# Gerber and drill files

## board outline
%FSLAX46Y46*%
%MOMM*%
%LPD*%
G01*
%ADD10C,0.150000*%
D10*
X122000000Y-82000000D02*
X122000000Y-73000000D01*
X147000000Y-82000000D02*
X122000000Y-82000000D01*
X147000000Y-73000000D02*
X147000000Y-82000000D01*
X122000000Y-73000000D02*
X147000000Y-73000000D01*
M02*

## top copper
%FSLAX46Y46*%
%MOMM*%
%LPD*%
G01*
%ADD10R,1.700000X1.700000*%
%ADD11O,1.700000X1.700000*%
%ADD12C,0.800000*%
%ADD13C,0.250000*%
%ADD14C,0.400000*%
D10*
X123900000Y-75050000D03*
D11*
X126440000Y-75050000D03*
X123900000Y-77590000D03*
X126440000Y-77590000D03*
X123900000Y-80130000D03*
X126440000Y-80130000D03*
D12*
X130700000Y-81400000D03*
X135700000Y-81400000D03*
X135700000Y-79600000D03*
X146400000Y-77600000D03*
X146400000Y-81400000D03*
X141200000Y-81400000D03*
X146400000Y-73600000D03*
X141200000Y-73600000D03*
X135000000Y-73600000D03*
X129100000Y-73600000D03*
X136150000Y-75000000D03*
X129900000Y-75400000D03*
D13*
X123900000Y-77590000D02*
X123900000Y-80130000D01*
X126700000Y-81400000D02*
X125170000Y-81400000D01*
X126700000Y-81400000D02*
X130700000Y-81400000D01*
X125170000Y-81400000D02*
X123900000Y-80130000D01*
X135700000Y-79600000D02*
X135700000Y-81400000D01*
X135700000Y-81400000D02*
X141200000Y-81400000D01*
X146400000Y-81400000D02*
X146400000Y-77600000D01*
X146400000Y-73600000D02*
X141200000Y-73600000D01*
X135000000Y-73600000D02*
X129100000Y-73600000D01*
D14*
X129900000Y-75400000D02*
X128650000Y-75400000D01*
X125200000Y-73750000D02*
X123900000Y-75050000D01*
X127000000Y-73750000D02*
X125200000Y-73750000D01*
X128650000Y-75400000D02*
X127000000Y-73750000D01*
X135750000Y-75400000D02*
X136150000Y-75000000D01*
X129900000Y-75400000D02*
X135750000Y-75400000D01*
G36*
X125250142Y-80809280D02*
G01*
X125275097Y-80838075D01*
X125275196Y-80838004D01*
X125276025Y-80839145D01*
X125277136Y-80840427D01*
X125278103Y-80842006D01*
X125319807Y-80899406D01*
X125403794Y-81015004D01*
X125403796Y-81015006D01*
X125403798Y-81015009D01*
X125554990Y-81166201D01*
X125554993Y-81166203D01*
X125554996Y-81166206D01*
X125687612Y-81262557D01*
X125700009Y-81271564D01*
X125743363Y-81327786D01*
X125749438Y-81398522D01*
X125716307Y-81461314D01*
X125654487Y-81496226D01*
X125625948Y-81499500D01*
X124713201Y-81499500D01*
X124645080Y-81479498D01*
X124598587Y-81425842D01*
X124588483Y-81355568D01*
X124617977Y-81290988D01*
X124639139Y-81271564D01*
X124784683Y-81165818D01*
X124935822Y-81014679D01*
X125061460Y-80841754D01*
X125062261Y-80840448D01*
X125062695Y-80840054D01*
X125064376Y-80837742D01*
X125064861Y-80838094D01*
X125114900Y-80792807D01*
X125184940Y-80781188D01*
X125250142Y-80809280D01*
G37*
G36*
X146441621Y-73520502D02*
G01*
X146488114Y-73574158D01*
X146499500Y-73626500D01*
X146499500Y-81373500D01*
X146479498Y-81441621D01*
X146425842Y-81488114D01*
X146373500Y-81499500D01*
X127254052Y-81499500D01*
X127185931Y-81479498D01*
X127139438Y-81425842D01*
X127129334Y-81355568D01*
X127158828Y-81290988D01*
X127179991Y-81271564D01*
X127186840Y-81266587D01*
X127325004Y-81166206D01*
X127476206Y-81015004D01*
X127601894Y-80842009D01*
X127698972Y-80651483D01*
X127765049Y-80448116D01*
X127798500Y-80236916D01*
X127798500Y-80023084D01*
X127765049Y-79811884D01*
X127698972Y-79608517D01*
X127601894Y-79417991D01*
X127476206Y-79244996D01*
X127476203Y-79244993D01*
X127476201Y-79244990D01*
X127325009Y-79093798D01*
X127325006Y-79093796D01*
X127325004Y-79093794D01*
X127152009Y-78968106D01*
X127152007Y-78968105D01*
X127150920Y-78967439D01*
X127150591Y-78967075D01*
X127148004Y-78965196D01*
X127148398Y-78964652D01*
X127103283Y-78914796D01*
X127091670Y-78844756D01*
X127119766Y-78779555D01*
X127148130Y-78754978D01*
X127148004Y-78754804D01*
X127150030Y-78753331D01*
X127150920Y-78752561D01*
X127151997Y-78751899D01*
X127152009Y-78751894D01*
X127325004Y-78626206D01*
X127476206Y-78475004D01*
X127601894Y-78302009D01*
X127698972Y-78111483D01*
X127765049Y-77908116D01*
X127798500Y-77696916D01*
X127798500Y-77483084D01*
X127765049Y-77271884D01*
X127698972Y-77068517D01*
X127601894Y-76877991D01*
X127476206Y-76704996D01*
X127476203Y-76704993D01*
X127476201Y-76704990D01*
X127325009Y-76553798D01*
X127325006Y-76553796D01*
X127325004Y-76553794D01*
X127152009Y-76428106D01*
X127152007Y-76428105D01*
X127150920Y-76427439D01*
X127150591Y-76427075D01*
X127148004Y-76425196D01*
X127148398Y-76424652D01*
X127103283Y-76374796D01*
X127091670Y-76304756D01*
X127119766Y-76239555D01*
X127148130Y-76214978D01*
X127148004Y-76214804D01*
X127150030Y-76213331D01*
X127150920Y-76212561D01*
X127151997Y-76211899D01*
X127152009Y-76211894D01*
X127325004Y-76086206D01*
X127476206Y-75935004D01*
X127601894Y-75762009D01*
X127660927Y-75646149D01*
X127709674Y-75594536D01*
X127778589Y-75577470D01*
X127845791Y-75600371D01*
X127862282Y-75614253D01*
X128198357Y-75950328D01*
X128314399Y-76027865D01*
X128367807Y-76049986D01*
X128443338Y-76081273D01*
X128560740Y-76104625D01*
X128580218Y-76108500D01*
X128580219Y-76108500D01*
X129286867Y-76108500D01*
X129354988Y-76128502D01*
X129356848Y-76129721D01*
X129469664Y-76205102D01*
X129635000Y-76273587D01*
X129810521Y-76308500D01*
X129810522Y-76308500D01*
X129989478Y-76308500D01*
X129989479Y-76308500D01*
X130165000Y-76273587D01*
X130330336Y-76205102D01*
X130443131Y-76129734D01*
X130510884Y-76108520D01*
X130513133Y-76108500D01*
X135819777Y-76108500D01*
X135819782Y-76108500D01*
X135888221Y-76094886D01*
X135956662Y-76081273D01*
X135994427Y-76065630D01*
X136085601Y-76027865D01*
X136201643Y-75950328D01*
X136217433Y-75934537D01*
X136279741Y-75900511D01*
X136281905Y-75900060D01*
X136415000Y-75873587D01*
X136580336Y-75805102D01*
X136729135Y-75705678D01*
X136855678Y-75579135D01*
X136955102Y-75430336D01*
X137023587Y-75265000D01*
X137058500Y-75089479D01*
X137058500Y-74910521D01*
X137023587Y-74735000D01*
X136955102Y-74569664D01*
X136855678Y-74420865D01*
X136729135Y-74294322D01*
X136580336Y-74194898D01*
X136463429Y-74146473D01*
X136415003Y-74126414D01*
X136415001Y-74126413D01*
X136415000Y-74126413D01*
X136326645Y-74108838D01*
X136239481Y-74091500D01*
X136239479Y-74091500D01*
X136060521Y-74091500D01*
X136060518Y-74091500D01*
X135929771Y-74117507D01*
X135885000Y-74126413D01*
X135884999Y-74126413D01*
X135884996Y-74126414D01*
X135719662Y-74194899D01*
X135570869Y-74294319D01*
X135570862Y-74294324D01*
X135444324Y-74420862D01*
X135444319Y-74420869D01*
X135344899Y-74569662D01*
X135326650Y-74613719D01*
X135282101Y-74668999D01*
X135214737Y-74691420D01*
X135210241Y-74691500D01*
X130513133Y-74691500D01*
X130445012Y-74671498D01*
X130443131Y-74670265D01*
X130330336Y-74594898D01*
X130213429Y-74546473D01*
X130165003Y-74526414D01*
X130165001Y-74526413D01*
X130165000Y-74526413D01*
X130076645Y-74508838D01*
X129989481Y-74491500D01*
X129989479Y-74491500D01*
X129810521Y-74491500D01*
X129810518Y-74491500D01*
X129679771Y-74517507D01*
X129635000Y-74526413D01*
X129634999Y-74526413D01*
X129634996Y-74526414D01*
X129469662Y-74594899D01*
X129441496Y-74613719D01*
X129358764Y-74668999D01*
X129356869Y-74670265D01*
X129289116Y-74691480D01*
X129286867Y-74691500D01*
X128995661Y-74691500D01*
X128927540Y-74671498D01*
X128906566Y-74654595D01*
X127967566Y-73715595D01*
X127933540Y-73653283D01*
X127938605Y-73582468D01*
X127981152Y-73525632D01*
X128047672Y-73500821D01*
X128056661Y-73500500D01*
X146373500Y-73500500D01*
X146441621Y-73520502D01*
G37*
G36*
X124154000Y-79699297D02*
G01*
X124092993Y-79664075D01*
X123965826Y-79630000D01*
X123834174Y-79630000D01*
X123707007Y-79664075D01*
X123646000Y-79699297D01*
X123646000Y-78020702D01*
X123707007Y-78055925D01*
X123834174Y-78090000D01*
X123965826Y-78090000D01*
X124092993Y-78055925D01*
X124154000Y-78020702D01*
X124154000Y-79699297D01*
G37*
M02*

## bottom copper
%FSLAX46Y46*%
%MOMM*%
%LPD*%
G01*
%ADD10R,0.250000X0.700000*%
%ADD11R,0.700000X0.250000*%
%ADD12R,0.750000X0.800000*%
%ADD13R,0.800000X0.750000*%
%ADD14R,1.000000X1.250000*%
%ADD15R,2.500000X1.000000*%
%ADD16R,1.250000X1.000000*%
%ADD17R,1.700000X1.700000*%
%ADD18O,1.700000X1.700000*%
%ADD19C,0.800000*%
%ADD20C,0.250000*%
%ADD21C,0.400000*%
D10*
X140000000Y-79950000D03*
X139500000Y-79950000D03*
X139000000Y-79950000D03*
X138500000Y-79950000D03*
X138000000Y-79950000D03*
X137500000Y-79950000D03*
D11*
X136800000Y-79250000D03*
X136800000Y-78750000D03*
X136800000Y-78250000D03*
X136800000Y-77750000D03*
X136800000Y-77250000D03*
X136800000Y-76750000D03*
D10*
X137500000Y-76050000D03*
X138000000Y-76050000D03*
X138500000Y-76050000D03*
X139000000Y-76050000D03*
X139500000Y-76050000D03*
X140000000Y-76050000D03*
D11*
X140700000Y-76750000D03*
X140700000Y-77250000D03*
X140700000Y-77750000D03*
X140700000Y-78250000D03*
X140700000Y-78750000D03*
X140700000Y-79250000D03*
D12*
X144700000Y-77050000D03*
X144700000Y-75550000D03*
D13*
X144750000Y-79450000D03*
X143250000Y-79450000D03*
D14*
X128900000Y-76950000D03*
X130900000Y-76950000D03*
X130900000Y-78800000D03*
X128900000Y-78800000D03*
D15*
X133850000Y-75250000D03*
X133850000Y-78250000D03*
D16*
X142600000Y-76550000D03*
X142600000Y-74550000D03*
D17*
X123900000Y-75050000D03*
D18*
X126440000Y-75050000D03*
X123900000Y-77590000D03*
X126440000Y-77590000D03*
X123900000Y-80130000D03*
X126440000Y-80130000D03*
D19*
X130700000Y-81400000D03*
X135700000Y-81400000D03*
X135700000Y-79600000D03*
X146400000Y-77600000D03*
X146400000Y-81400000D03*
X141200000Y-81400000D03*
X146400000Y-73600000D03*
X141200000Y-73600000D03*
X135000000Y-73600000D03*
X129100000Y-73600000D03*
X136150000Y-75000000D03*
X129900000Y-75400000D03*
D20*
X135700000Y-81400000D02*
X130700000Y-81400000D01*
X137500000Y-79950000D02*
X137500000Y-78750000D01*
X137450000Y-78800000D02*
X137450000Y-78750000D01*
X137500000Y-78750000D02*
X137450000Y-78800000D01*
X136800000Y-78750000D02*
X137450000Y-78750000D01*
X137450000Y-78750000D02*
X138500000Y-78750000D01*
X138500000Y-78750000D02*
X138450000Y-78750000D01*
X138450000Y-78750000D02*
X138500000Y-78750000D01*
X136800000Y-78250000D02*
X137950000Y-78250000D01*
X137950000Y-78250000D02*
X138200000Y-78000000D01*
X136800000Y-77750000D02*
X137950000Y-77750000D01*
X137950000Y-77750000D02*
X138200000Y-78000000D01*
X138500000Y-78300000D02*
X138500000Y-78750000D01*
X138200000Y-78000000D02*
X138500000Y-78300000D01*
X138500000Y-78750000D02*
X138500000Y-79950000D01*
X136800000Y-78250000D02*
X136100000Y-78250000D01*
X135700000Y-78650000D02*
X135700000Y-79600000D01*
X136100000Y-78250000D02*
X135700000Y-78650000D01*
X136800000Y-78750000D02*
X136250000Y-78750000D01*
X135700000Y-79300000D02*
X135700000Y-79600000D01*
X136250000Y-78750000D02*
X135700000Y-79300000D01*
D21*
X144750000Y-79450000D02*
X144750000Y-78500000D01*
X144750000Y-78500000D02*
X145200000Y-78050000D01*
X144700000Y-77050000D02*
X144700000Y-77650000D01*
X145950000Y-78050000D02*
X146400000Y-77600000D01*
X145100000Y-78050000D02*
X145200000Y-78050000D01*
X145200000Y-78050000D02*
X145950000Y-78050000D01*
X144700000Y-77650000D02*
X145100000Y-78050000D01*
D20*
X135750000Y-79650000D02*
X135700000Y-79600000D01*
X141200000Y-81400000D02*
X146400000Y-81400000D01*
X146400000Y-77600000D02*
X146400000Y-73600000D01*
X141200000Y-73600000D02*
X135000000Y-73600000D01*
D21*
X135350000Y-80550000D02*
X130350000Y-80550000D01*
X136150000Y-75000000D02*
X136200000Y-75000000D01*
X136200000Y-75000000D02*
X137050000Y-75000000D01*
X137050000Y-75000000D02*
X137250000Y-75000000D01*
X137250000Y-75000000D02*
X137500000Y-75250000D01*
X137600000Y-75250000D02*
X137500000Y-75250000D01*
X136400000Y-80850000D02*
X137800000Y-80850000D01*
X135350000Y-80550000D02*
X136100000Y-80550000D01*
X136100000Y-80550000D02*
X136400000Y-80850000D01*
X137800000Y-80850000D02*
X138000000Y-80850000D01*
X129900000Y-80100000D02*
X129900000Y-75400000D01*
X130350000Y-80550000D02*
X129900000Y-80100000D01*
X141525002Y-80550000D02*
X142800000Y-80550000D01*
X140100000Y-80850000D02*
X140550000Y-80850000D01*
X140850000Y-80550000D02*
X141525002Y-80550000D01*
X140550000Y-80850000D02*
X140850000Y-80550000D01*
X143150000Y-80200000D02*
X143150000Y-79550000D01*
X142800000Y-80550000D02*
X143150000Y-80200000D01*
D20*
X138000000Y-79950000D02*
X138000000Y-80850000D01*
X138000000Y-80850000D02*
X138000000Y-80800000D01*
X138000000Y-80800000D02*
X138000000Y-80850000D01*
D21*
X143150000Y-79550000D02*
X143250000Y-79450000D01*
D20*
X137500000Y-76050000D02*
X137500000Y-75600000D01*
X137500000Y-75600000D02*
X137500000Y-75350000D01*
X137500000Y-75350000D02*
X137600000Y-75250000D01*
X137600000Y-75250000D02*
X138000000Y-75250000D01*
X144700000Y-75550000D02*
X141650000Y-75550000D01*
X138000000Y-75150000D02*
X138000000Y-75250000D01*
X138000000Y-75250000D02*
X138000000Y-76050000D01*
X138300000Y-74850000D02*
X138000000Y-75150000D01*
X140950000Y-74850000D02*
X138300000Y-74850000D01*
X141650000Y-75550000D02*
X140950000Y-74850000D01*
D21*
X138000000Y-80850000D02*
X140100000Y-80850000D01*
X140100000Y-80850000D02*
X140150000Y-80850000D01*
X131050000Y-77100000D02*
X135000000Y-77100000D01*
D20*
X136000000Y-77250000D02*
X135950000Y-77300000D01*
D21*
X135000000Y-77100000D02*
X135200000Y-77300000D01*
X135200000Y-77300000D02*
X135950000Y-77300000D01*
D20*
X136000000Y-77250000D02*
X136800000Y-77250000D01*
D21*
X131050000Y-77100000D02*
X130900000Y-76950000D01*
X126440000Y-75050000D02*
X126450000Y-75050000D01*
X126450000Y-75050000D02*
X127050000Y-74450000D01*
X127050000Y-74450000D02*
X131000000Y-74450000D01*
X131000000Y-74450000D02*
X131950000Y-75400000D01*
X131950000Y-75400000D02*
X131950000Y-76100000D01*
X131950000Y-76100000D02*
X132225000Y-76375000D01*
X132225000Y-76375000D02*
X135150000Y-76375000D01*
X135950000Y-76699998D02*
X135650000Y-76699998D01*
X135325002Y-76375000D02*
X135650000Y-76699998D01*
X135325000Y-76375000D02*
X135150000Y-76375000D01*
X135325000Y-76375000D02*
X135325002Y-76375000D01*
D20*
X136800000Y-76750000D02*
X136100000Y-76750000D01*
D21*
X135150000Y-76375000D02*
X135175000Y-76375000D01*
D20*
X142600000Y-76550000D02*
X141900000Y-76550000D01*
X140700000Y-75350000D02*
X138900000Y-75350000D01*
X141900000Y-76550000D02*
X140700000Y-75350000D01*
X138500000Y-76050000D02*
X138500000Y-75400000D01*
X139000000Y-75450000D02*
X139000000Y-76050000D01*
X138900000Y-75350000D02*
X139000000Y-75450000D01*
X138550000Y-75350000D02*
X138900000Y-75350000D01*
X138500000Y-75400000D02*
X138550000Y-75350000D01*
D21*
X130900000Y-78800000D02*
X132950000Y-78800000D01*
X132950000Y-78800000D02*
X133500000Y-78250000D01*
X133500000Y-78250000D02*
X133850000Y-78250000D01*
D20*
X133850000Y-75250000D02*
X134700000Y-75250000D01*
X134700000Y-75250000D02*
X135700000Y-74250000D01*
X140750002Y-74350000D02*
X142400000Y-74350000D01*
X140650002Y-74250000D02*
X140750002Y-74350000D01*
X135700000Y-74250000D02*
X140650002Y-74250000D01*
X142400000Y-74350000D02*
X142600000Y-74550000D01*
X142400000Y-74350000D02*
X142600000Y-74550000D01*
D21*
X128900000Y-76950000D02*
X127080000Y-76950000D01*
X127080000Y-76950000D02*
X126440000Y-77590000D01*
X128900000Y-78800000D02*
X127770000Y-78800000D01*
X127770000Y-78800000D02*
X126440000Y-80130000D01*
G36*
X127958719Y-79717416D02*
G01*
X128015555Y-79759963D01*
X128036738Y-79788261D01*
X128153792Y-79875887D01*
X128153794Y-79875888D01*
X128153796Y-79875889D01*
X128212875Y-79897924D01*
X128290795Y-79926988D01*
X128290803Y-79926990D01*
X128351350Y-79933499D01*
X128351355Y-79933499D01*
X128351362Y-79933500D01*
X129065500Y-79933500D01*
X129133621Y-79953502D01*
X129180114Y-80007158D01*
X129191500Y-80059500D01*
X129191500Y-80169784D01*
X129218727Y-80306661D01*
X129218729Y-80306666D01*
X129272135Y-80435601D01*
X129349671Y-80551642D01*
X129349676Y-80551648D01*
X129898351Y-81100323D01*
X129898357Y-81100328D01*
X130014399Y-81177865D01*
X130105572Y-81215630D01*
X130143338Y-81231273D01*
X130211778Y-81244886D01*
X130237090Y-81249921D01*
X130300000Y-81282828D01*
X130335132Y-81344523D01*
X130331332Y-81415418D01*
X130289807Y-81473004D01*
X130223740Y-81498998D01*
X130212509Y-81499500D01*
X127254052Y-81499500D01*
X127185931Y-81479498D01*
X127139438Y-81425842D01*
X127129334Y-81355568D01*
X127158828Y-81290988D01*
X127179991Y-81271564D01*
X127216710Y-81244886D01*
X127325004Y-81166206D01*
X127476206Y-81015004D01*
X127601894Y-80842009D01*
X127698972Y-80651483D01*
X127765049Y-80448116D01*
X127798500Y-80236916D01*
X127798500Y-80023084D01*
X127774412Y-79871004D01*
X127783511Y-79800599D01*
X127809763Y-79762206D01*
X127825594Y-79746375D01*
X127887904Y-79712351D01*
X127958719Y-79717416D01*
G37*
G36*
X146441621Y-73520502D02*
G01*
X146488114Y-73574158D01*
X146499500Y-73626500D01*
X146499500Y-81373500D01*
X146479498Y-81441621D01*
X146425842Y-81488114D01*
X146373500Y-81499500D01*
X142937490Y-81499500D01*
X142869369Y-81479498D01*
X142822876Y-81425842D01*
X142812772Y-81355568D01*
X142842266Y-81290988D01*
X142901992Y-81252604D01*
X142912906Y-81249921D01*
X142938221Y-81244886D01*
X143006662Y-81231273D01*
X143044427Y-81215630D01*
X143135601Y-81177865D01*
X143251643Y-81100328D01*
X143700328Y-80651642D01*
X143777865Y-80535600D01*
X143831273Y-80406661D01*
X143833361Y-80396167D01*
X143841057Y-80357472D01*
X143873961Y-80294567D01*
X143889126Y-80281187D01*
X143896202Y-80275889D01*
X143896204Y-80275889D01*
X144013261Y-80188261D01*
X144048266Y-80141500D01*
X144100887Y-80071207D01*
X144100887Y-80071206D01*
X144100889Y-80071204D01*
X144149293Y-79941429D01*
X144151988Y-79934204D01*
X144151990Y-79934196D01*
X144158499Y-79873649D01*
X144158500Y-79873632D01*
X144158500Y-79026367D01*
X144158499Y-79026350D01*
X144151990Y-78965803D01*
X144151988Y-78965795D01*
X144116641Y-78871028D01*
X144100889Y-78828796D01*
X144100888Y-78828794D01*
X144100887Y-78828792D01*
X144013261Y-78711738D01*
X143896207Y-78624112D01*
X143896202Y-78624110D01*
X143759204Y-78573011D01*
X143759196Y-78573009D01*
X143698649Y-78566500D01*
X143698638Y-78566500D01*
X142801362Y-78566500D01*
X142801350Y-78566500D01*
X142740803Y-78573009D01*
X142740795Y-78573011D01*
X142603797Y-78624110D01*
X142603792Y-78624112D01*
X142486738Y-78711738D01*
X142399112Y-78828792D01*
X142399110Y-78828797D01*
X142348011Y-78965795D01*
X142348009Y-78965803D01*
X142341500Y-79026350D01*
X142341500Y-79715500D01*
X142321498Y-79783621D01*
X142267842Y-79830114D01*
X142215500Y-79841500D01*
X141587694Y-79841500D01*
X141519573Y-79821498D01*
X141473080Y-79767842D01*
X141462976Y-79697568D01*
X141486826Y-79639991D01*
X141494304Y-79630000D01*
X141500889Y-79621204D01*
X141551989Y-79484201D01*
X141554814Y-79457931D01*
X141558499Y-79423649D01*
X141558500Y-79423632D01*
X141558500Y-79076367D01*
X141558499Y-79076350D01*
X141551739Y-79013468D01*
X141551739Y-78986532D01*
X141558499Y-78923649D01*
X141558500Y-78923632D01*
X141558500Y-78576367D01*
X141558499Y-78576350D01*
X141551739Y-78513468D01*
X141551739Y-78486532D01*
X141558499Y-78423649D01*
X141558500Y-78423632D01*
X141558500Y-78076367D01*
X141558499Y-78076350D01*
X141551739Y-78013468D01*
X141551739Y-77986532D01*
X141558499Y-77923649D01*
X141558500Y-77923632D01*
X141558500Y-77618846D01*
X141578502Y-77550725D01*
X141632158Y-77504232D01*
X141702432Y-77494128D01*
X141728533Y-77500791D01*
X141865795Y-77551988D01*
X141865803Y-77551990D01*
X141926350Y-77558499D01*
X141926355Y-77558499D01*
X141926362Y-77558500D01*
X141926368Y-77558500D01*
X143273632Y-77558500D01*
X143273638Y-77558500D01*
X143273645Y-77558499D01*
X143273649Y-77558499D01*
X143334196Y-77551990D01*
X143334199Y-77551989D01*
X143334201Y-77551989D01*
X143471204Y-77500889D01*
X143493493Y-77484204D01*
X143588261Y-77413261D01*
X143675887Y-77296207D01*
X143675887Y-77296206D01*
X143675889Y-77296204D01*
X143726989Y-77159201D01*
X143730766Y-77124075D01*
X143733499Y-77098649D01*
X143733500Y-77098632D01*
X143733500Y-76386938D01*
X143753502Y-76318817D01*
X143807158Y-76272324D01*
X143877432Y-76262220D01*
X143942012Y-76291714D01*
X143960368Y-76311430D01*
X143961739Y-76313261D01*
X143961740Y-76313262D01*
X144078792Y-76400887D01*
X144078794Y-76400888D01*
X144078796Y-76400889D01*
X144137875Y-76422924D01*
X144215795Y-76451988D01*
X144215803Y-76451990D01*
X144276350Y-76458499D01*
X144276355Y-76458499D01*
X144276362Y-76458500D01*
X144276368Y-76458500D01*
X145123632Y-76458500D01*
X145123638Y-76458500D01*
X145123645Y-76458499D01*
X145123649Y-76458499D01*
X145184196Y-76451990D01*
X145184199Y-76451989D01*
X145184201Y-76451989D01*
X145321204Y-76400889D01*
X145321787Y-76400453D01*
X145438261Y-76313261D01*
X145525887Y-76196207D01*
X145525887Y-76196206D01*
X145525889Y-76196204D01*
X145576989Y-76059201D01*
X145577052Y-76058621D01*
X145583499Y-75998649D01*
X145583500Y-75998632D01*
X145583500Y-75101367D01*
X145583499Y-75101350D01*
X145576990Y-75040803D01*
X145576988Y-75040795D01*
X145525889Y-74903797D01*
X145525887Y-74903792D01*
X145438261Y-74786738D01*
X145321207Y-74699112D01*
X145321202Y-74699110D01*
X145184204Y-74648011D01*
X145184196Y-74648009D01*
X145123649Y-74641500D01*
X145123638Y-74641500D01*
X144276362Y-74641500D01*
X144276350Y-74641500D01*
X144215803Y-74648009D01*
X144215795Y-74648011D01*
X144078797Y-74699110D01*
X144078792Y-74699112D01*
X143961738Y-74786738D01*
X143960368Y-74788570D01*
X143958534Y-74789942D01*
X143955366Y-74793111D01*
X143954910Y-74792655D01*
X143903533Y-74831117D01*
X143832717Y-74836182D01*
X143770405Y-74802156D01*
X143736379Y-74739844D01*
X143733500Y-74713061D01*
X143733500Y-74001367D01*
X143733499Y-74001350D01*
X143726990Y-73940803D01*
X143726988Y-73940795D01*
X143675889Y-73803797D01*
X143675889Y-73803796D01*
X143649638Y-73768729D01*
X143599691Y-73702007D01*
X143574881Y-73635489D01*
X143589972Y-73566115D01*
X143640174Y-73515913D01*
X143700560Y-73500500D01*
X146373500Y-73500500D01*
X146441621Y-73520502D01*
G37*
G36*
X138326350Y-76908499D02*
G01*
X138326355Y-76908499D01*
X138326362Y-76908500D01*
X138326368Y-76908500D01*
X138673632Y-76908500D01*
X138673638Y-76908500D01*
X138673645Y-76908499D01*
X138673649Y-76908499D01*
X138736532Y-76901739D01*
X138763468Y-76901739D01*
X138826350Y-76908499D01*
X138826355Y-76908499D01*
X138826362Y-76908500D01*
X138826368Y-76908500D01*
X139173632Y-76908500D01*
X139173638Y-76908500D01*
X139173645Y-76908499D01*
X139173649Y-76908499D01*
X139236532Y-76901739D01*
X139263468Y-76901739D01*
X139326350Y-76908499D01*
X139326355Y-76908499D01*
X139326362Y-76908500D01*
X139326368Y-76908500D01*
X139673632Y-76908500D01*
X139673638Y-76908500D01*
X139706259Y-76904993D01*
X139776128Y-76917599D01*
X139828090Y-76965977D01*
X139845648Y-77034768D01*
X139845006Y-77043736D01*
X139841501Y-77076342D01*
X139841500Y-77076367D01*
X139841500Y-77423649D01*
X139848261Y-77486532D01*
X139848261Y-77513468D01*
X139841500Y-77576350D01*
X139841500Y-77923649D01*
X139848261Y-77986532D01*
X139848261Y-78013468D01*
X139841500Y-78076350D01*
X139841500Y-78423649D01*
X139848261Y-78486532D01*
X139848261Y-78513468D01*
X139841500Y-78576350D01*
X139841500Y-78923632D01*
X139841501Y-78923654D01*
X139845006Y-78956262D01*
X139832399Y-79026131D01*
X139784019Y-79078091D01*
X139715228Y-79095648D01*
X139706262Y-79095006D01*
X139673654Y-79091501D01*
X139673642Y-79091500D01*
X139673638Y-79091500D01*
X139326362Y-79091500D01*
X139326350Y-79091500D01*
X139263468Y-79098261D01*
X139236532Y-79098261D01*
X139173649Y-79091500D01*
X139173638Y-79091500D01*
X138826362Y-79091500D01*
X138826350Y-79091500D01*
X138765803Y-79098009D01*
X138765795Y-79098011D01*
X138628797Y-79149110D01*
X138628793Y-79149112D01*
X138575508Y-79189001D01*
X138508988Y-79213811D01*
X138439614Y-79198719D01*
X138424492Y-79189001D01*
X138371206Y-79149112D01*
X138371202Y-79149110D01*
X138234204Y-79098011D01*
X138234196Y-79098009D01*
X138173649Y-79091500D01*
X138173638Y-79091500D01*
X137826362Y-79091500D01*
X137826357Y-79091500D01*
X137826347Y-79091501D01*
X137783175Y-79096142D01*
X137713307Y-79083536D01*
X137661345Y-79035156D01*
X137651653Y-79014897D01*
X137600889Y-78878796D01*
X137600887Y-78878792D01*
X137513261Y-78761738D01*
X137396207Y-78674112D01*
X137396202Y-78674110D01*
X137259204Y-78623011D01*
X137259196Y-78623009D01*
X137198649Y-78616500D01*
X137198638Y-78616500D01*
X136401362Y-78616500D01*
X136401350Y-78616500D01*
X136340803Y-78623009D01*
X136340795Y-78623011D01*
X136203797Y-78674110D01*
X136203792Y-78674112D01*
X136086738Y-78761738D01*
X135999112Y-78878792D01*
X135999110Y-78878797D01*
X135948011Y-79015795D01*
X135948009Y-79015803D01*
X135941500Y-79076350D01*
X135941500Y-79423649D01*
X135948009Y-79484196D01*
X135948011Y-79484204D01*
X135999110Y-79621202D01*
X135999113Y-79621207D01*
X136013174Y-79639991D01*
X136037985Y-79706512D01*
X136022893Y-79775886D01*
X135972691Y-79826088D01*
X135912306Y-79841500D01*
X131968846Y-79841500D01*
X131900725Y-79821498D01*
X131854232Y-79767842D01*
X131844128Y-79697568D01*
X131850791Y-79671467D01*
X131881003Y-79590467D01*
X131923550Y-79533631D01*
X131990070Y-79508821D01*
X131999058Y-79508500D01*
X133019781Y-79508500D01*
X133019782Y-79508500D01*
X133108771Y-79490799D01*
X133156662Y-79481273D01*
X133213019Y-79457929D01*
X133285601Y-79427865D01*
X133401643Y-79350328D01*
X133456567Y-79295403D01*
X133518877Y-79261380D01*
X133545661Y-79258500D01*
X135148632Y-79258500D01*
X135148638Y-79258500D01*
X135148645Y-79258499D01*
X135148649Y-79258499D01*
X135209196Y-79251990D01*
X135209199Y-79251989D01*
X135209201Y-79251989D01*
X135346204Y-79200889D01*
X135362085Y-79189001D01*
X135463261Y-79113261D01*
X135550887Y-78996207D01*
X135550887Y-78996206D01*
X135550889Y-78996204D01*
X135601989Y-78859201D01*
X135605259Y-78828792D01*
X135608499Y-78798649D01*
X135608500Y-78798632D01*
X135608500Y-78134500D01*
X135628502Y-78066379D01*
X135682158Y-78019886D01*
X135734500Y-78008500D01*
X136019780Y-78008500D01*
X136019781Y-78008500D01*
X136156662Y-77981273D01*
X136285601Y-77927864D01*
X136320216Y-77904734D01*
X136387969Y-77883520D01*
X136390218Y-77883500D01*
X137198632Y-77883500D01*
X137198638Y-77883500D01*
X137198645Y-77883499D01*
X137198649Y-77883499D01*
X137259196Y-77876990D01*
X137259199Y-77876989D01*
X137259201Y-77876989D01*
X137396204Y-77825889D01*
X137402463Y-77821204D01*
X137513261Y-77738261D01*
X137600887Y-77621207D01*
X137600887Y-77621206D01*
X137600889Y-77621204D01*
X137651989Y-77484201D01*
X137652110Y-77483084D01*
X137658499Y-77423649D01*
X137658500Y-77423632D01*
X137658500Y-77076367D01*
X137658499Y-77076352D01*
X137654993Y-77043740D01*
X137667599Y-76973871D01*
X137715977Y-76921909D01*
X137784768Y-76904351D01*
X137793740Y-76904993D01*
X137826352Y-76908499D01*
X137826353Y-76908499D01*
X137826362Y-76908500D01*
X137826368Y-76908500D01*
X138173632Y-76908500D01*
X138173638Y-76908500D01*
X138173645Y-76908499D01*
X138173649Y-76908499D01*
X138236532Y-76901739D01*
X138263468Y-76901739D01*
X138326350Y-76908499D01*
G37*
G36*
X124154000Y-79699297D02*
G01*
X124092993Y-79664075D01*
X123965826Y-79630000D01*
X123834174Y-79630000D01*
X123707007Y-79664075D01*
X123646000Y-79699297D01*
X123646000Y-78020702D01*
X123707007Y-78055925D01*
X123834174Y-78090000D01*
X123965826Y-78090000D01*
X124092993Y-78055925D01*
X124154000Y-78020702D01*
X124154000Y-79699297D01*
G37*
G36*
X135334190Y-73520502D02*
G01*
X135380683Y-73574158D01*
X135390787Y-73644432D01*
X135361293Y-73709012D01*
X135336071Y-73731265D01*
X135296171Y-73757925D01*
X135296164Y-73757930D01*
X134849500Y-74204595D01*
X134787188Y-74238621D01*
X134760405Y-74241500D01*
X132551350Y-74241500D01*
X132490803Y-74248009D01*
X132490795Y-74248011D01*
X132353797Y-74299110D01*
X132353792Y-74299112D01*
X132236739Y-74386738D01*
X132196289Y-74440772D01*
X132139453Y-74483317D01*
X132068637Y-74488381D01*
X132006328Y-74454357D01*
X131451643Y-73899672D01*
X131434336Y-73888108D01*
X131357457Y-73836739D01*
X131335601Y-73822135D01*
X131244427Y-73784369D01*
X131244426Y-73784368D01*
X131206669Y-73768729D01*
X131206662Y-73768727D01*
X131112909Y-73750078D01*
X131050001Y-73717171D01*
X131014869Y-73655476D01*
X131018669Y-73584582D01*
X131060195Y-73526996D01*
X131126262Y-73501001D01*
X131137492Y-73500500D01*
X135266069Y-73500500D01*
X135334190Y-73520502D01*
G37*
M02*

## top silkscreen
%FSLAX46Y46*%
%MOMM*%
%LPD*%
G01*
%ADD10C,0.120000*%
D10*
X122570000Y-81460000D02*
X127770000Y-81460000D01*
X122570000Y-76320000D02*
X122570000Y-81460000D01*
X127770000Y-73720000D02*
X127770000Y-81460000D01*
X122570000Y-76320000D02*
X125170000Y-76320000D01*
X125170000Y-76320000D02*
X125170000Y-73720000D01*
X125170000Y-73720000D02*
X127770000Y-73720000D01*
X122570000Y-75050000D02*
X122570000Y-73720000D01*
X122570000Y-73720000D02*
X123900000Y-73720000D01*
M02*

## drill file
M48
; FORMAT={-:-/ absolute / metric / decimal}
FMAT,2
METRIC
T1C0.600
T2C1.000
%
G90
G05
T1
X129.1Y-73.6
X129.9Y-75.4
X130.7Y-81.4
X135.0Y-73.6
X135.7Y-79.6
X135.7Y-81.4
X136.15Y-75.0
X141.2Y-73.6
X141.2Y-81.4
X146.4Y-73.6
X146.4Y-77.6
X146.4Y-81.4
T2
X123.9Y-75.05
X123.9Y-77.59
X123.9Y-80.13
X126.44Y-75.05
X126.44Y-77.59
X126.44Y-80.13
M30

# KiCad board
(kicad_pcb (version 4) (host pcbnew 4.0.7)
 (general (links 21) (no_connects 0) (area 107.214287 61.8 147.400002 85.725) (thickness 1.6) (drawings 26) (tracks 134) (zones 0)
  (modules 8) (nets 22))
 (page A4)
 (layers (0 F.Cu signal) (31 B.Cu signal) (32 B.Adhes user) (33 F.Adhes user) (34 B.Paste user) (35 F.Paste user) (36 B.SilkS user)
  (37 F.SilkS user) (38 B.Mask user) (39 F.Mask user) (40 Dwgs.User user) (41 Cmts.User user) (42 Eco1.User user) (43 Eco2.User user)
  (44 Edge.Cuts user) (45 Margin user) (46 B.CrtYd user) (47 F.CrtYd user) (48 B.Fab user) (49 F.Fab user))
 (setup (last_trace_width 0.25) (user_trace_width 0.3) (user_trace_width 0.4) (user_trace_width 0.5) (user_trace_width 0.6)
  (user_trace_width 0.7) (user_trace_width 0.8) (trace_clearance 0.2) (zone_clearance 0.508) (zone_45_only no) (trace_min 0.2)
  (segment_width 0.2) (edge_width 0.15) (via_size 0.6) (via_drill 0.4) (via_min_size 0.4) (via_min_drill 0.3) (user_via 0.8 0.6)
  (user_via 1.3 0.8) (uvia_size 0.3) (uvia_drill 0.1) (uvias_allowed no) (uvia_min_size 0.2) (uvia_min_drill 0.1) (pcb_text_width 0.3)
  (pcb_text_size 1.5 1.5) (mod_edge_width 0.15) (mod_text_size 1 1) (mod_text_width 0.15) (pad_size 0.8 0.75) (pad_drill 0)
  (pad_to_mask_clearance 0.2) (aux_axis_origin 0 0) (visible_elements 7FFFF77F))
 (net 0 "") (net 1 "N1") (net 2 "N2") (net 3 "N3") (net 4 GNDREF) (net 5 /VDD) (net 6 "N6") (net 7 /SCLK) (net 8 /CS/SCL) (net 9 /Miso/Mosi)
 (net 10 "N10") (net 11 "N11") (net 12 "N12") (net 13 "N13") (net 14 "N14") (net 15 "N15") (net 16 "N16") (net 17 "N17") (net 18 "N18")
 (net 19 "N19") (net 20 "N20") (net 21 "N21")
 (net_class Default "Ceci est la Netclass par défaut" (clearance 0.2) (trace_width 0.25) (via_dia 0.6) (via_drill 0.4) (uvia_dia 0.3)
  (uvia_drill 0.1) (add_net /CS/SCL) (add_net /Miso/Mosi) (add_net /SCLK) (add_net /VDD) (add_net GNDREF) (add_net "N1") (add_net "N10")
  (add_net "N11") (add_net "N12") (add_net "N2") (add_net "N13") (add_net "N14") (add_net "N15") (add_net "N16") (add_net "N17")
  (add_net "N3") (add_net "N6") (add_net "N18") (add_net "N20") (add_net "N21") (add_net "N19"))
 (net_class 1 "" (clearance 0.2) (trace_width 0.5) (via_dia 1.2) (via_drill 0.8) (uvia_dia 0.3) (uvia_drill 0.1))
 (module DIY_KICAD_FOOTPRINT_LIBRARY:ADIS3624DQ (layer B.Cu) (at 138.75 78 90)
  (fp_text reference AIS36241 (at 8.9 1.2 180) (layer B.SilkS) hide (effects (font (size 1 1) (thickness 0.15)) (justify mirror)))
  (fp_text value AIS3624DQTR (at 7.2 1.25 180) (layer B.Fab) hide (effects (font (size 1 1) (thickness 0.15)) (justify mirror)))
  (pad 1 smd rect (at -1.95 1.25 90) (size 0.7 0.25) (layers B.Cu B.Paste B.Mask) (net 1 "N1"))
  (pad 2 smd rect (at -1.95 0.75 90) (size 0.7 0.25) (layers B.Cu B.Paste B.Mask) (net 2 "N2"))
  (pad 3 smd rect (at -1.95 0.25 90) (size 0.7 0.25) (layers B.Cu B.Paste B.Mask) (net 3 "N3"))
  (pad 4 smd rect (at -1.95 -0.25 90) (size 0.7 0.25) (layers B.Cu B.Paste B.Mask) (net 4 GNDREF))
  (pad 5 smd rect (at -1.95 -0.75 90) (size 0.7 0.25) (layers B.Cu B.Paste B.Mask) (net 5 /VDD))
  (pad 6 smd rect (at -1.95 -1.25 90) (size 0.7 0.25) (layers B.Cu B.Paste B.Mask) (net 4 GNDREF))
  (pad 7 smd rect (at -1.25 -1.95 180) (size 0.7 0.25) (layers B.Cu B.Paste B.Mask) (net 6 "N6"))
  (pad 8 smd rect (at -0.75 -1.95 180) (size 0.7 0.25) (layers B.Cu B.Paste B.Mask) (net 4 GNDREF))
  (pad 9 smd rect (at -0.25 -1.95 180) (size 0.7 0.25) (layers B.Cu B.Paste B.Mask) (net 4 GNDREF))
  (pad 10 smd rect (at 0.25 -1.95 180) (size 0.7 0.25) (layers B.Cu B.Paste B.Mask) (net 4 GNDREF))
  (pad 11 smd rect (at 0.75 -1.95 180) (size 0.7 0.25) (layers B.Cu B.Paste B.Mask) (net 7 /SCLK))
  (pad 12 smd rect (at 1.25 -1.95 180) (size 0.7 0.25) (layers B.Cu B.Paste B.Mask) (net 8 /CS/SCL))
  (pad 13 smd rect (at 1.95 -1.25 90) (size 0.7 0.25) (layers B.Cu B.Paste B.Mask) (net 5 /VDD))
  (pad 14 smd rect (at 1.95 -0.75 90) (size 0.7 0.25) (layers B.Cu B.Paste B.Mask) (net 5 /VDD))
  (pad 15 smd rect (at 1.95 -0.25 90) (size 0.7 0.25) (layers B.Cu B.Paste B.Mask) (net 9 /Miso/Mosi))
  (pad 16 smd rect (at 1.95 0.25 90) (size 0.7 0.25) (layers B.Cu B.Paste B.Mask) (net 9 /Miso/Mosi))
  (pad 17 smd rect (at 1.95 0.75 90) (size 0.7 0.25) (layers B.Cu B.Paste B.Mask) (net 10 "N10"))
  (pad 18 smd rect (at 1.95 1.25 90) (size 0.7 0.25) (layers B.Cu B.Paste B.Mask) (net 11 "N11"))
  (pad 19 smd rect (at 1.25 1.95) (size 0.7 0.25) (layers B.Cu B.Paste B.Mask) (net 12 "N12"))
  (pad 20 smd rect (at 0.75 1.95) (size 0.7 0.25) (layers B.Cu B.Paste B.Mask) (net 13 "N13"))
  (pad 21 smd rect (at 0.25 1.95) (size 0.7 0.25) (layers B.Cu B.Paste B.Mask) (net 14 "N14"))
  (pad 22 smd rect (at -0.25 1.95) (size 0.7 0.25) (layers B.Cu B.Paste B.Mask) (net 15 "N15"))
  (pad 23 smd rect (at -0.75 1.95) (size 0.7 0.25) (layers B.Cu B.Paste B.Mask) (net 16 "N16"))
  (pad 24 smd rect (at -1.25 1.95) (size 0.7 0.25) (layers B.Cu B.Paste B.Mask) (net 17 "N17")))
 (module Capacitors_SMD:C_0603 (layer B.Cu) (at 144.7 76.3 270)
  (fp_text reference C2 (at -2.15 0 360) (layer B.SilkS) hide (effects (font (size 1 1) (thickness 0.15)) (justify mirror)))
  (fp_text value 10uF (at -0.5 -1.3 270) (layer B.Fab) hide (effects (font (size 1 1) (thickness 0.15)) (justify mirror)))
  (pad 2 smd rect (at 0.75 0 270) (size 0.8 0.75) (layers B.Cu B.Paste B.Mask) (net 4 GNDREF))
  (pad 1 smd rect (at -0.75 0 270) (size 0.8 0.75) (layers B.Cu B.Paste B.Mask) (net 5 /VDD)))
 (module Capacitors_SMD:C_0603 (layer B.Cu) (at 144 79.45)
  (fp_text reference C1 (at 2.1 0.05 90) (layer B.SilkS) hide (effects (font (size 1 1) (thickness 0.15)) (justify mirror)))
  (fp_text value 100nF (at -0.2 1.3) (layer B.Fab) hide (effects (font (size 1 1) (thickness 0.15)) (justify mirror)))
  (pad 2 smd rect (at 0.75 0) (size 0.8 0.75) (layers B.Cu B.Paste B.Mask) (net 4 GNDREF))
  (pad 1 smd rect (at -0.75 0) (size 0.8 0.75) (layers B.Cu B.Paste B.Mask) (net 5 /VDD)))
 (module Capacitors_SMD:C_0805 (layer B.Cu) (at 129.9 76.95)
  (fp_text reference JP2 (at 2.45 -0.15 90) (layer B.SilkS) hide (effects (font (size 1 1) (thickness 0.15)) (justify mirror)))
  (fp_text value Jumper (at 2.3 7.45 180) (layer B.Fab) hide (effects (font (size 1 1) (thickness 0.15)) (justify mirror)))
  (pad 1 smd rect (at -1 0) (size 1 1.25) (layers B.Cu B.Paste B.Mask) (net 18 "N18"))
  (pad 2 smd rect (at 1 0) (size 1 1.25) (layers B.Cu B.Paste B.Mask) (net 7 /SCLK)))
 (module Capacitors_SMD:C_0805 (layer B.Cu) (at 129.9 78.8 180)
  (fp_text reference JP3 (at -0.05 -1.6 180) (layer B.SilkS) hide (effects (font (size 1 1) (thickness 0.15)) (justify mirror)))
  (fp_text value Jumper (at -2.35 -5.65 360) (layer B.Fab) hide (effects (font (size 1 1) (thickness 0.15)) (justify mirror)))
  (pad 1 smd rect (at -1 0 180) (size 1 1.25) (layers B.Cu B.Paste B.Mask) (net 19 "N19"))
  (pad 2 smd rect (at 1 0 180) (size 1 1.25) (layers B.Cu B.Paste B.Mask) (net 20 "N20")))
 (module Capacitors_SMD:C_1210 (layer B.Cu) (at 133.85 76.75 270)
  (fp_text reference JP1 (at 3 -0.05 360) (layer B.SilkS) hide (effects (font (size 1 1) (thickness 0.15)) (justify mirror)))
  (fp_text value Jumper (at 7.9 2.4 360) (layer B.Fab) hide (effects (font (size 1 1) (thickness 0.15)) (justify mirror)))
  (pad 1 smd rect (at -1.5 0 270) (size 1 2.5) (layers B.Cu B.Paste B.Mask) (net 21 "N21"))
  (pad 2 smd rect (at 1.5 0 270) (size 1 2.5) (layers B.Cu B.Paste B.Mask) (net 19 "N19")))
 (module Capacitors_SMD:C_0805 (layer B.Cu) (at 142.6 75.55 90)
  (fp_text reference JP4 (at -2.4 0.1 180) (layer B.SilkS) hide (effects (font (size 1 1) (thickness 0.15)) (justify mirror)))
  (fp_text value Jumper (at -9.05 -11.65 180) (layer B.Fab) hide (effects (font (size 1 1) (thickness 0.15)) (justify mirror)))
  (pad 1 smd rect (at -1 0 90) (size 1 1.25) (layers B.Cu B.Paste B.Mask) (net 9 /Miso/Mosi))
  (pad 2 smd rect (at 1 0 90) (size 1 1.25) (layers B.Cu B.Paste B.Mask) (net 21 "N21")))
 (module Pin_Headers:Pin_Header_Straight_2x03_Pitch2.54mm (layer F.Cu) (at 123.9 75.05)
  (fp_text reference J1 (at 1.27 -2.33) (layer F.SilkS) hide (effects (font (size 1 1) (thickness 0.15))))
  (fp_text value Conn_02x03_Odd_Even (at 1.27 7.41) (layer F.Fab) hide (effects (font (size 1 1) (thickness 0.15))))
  (fp_line (start -1.33 6.41) (end 3.87 6.41) (layer F.SilkS) (width 0.12))
  (fp_line (start -1.33 1.27) (end -1.33 6.41) (layer F.SilkS) (width 0.12))
  (fp_line (start 3.87 -1.33) (end 3.87 6.41) (layer F.SilkS) (width 0.12))
  (fp_line (start -1.33 1.27) (end 1.27 1.27) (layer F.SilkS) (width 0.12))
  (fp_line (start 1.27 1.27) (end 1.27 -1.33) (layer F.SilkS) (width 0.12))
  (fp_line (start 1.27 -1.33) (end 3.87 -1.33) (layer F.SilkS) (width 0.12))
  (fp_line (start -1.33 0) (end -1.33 -1.33) (layer F.SilkS) (width 0.12))
  (fp_line (start -1.33 -1.33) (end 0 -1.33) (layer F.SilkS) (width 0.12))
  (pad 1 thru_hole rect (at 0 0) (size 1.7 1.7) (drill 1) (layers *.Cu *.Mask) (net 5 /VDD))
  (pad 2 thru_hole oval (at 2.54 0) (size 1.7 1.7) (drill 1) (layers *.Cu *.Mask) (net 8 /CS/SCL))
  (pad 3 thru_hole oval (at 0 2.54) (size 1.7 1.7) (drill 1) (layers *.Cu *.Mask) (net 4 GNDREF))
  (pad 4 thru_hole oval (at 2.54 2.54) (size 1.7 1.7) (drill 1) (layers *.Cu *.Mask) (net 18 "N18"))
  (pad 5 thru_hole oval (at 0 5.08) (size 1.7 1.7) (drill 1) (layers *.Cu *.Mask) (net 4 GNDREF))
  (pad 6 thru_hole oval (at 2.54 5.08) (size 1.7 1.7) (drill 1) (layers *.Cu *.Mask) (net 20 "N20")))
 (gr_line (start 122 82) (end 122 73) (angle 90) (layer Edge.Cuts) (width 0.15))
 (gr_line (start 147 82) (end 122 82) (angle 90) (layer Edge.Cuts) (width 0.15))
 (gr_line (start 147 73) (end 147 82) (angle 90) (layer Edge.Cuts) (width 0.15))
 (gr_line (start 122 73) (end 147 73) (angle 90) (layer Edge.Cuts) (width 0.15))
 (segment (start 123.9 77.59) (end 123.9 80.13) (width 0.25) (layer F.Cu) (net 4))
 (segment (start 126.7 81.4) (end 125.17 81.4) (width 0.25) (layer F.Cu) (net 4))
 (segment (start 126.7 81.4) (end 130.7 81.4) (width 0.25) (layer F.Cu) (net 4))
 (via (at 130.7 81.4) (size 0.8) (drill 0.6) (layers F.Cu B.Cu) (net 4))
 (segment (start 135.7 81.4) (end 130.7 81.4) (width 0.25) (layer B.Cu) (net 4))
 (via (at 135.7 81.4) (size 0.8) (drill 0.6) (layers F.Cu B.Cu) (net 4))
 (segment (start 125.17 81.4) (end 123.9 80.13) (width 0.25) (layer F.Cu) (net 4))
 (segment (start 137.5 79.95) (end 137.5 78.75) (width 0.25) (layer B.Cu) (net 4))
 (segment (start 137.45 78.8) (end 137.45 78.75) (width 0.25) (layer B.Cu) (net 4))
 (segment (start 137.5 78.75) (end 137.45 78.8) (width 0.25) (layer B.Cu) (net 4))
 (segment (start 136.8 78.75) (end 137.45 78.75) (width 0.25) (layer B.Cu) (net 4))
 (segment (start 137.45 78.75) (end 138.5 78.75) (width 0.25) (layer B.Cu) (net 4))
 (segment (start 138.5 78.75) (end 138.45 78.75) (width 0.25) (layer B.Cu) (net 4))
 (segment (start 138.45 78.75) (end 138.5 78.75) (width 0.25) (layer B.Cu) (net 4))
 (segment (start 136.8 78.25) (end 137.95 78.25) (width 0.25) (layer B.Cu) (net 4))
 (segment (start 137.95 78.25) (end 138.2 78) (width 0.25) (layer B.Cu) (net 4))
 (segment (start 136.8 77.75) (end 137.95 77.75) (width 0.25) (layer B.Cu) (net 4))
 (segment (start 137.95 77.75) (end 138.2 78) (width 0.25) (layer B.Cu) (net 4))
 (segment (start 138.5 78.3) (end 138.5 78.75) (width 0.25) (layer B.Cu) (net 4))
 (segment (start 138.2 78) (end 138.5 78.3) (width 0.25) (layer B.Cu) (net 4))
 (segment (start 138.5 78.75) (end 138.5 79.95) (width 0.25) (layer B.Cu) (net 4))
 (segment (start 136.8 78.25) (end 136.1 78.25) (width 0.25) (layer B.Cu) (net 4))
 (segment (start 135.7 78.65) (end 135.7 79.6) (width 0.25) (layer B.Cu) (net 4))
 (segment (start 136.1 78.25) (end 135.7 78.65) (width 0.25) (layer B.Cu) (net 4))
 (segment (start 136.8 78.75) (end 136.25 78.75) (width 0.25) (layer B.Cu) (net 4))
 (segment (start 135.7 79.3) (end 135.7 79.6) (width 0.25) (layer B.Cu) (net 4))
 (segment (start 136.25 78.75) (end 135.7 79.3) (width 0.25) (layer B.Cu) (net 4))
 (segment (start 144.75 79.45) (end 144.75 78.5) (width 0.4) (layer B.Cu) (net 4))
 (segment (start 144.75 78.5) (end 145.2 78.05) (width 0.4) (layer B.Cu) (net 4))
 (segment (start 144.7 77.05) (end 144.7 77.65) (width 0.4) (layer B.Cu) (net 4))
 (segment (start 145.95 78.05) (end 146.4 77.6) (width 0.4) (layer B.Cu) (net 4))
 (segment (start 145.1 78.05) (end 145.2 78.05) (width 0.4) (layer B.Cu) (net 4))
 (segment (start 145.2 78.05) (end 145.95 78.05) (width 0.4) (layer B.Cu) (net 4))
 (segment (start 144.7 77.65) (end 145.1 78.05) (width 0.4) (layer B.Cu) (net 4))
 (segment (start 135.75 79.65) (end 135.7 79.6) (width 0.25) (layer B.Cu) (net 4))
 (via (at 135.7 79.6) (size 0.8) (drill 0.6) (layers F.Cu B.Cu) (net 4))
 (segment (start 135.7 79.6) (end 135.7 81.4) (width 0.25) (layer F.Cu) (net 4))
 (segment (start 135.7 81.4) (end 141.2 81.4) (width 0.25) (layer F.Cu) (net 4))
 (via (at 146.4 77.6) (size 0.8) (drill 0.6) (layers F.Cu B.Cu) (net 4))
 (segment (start 146.4 81.4) (end 146.4 77.6) (width 0.25) (layer F.Cu) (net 4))
 (via (at 146.4 81.4) (size 0.8) (drill 0.6) (layers F.Cu B.Cu) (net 4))
 (segment (start 141.2 81.4) (end 146.4 81.4) (width 0.25) (layer B.Cu) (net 4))
 (via (at 141.2 81.4) (size 0.8) (drill 0.6) (layers F.Cu B.Cu) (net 4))
 (segment (start 146.4 77.6) (end 146.4 73.6) (width 0.25) (layer B.Cu) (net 4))
 (via (at 146.4 73.6) (size 0.8) (drill 0.6) (layers F.Cu B.Cu) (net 4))
 (segment (start 146.4 73.6) (end 141.2 73.6) (width 0.25) (layer F.Cu) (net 4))
 (via (at 141.2 73.6) (size 0.8) (drill 0.6) (layers F.Cu B.Cu) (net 4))
 (segment (start 141.2 73.6) (end 135 73.6) (width 0.25) (layer B.Cu) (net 4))
 (via (at 135 73.6) (size 0.8) (drill 0.6) (layers F.Cu B.Cu) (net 4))
 (segment (start 135 73.6) (end 129.1 73.6) (width 0.25) (layer F.Cu) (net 4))
 (via (at 129.1 73.6) (size 0.8) (drill 0.6) (layers F.Cu B.Cu) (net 4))
 (segment (start 129.9 75.4) (end 128.65 75.4) (width 0.4) (layer F.Cu) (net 5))
 (segment (start 125.2 73.75) (end 123.9 75.05) (width 0.4) (layer F.Cu) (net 5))
 (segment (start 127 73.75) (end 125.2 73.75) (width 0.4) (layer F.Cu) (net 5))
 (segment (start 128.65 75.4) (end 127 73.75) (width 0.4) (layer F.Cu) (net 5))
 (segment (start 135.35 80.55) (end 130.35 80.55) (width 0.4) (layer B.Cu) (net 5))
 (segment (start 135.75 75.4) (end 136.15 75) (width 0.4) (layer F.Cu) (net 5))
 (via (at 136.15 75) (size 0.8) (drill 0.6) (layers F.Cu B.Cu) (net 5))
 (segment (start 136.15 75) (end 136.2 75) (width 0.4) (layer B.Cu) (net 5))
 (segment (start 136.2 75) (end 137.05 75) (width 0.4) (layer B.Cu) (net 5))
 (segment (start 137.05 75) (end 137.25 75) (width 0.4) (layer B.Cu) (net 5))
 (segment (start 137.25 75) (end 137.5 75.25) (width 0.4) (layer B.Cu) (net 5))
 (segment (start 137.6 75.25) (end 137.5 75.25) (width 0.4) (layer B.Cu) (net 5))
 (segment (start 136.4 80.85) (end 137.8 80.85) (width 0.4) (layer B.Cu) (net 5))
 (segment (start 135.35 80.55) (end 136.1 80.55) (width 0.4) (layer B.Cu) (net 5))
 (segment (start 136.1 80.55) (end 136.4 80.85) (width 0.4) (layer B.Cu) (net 5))
 (segment (start 137.8 80.85) (end 138 80.85) (width 0.4) (layer B.Cu) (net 5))
 (segment (start 129.9 75.4) (end 135.75 75.4) (width 0.4) (layer F.Cu) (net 5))
 (via (at 129.9 75.4) (size 0.8) (drill 0.6) (layers F.Cu B.Cu) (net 5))
 (segment (start 129.9 80.1) (end 129.9 75.4) (width 0.4) (layer B.Cu) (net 5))
 (segment (start 130.35 80.55) (end 129.9 80.1) (width 0.4) (layer B.Cu) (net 5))
 (segment (start 141.525002 80.55) (end 142.8 80.55) (width 0.4) (layer B.Cu) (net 5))
 (segment (start 140.1 80.85) (end 140.55 80.85) (width 0.4) (layer B.Cu) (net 5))
 (segment (start 140.85 80.55) (end 141.525002 80.55) (width 0.4) (layer B.Cu) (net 5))
 (segment (start 140.55 80.85) (end 140.85 80.55) (width 0.4) (layer B.Cu) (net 5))
 (segment (start 143.15 80.2) (end 143.15 79.55) (width 0.4) (layer B.Cu) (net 5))
 (segment (start 142.8 80.55) (end 143.15 80.2) (width 0.4) (layer B.Cu) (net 5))
 (segment (start 138 79.95) (end 138 80.85) (width 0.25) (layer B.Cu) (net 5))
 (segment (start 138 80.85) (end 138 80.8) (width 0.25) (layer B.Cu) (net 5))
 (segment (start 138 80.8) (end 138 80.85) (width 0.25) (layer B.Cu) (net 5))
 (segment (start 143.15 79.55) (end 143.25 79.45) (width 0.4) (layer B.Cu) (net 5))
 (segment (start 137.5 76.05) (end 137.5 75.6) (width 0.25) (layer B.Cu) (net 5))
 (segment (start 137.5 75.6) (end 137.5 75.35) (width 0.25) (layer B.Cu) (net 5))
 (segment (start 137.5 75.35) (end 137.6 75.25) (width 0.25) (layer B.Cu) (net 5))
 (segment (start 137.6 75.25) (end 138 75.25) (width 0.25) (layer B.Cu) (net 5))
 (segment (start 144.7 75.55) (end 141.65 75.55) (width 0.25) (layer B.Cu) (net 5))
 (segment (start 138 75.15) (end 138 75.25) (width 0.25) (layer B.Cu) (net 5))
 (segment (start 138 75.25) (end 138 76.05) (width 0.25) (layer B.Cu) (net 5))
 (segment (start 138.3 74.85) (end 138 75.15) (width 0.25) (layer B.Cu) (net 5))
 (segment (start 140.95 74.85) (end 138.3 74.85) (width 0.25) (layer B.Cu) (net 5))
 (segment (start 141.65 75.55) (end 140.95 74.85) (width 0.25) (layer B.Cu) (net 5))
 (segment (start 138 80.85) (end 140.1 80.85) (width 0.4) (layer B.Cu) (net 5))
 (segment (start 140.1 80.85) (end 140.15 80.85) (width 0.4) (layer B.Cu) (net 5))
 (segment (start 131.05 77.1) (end 135 77.1) (width 0.4) (layer B.Cu) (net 7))
 (segment (start 136 77.25) (end 135.95 77.3) (width 0.25) (layer B.Cu) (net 7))
 (segment (start 135 77.1) (end 135.2 77.3) (width 0.4) (layer B.Cu) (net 7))
 (segment (start 135.2 77.3) (end 135.95 77.3) (width 0.4) (layer B.Cu) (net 7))
 (segment (start 136 77.25) (end 136.8 77.25) (width 0.25) (layer B.Cu) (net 7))
 (segment (start 131.05 77.1) (end 130.9 76.95) (width 0.4) (layer B.Cu) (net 7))
 (segment (start 126.44 75.05) (end 126.45 75.05) (width 0.4) (layer B.Cu) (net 8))
 (segment (start 126.45 75.05) (end 127.05 74.45) (width 0.4) (layer B.Cu) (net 8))
 (segment (start 127.05 74.45) (end 131 74.45) (width 0.4) (layer B.Cu) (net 8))
 (segment (start 131 74.45) (end 131.95 75.4) (width 0.4) (layer B.Cu) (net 8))
 (segment (start 131.95 75.4) (end 131.95 76.1) (width 0.4) (layer B.Cu) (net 8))
 (segment (start 131.95 76.1) (end 132.225 76.375) (width 0.4) (layer B.Cu) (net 8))
 (segment (start 132.225 76.375) (end 135.15 76.375) (width 0.4) (layer B.Cu) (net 8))
 (segment (start 135.95 76.699998) (end 135.65 76.699998) (width 0.4) (layer B.Cu) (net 8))
 (segment (start 135.325002 76.375) (end 135.65 76.699998) (width 0.4) (layer B.Cu) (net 8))
 (segment (start 135.325 76.375) (end 135.15 76.375) (width 0.4) (layer B.Cu) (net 8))
 (segment (start 135.325 76.375) (end 135.325002 76.375) (width 0.4) (layer B.Cu) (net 8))
 (segment (start 136.8 76.75) (end 136.1 76.75) (width 0.25) (layer B.Cu) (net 8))
 (segment (start 135.15 76.375) (end 135.175 76.375) (width 0.4) (layer B.Cu) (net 8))
 (segment (start 142.6 76.55) (end 141.9 76.55) (width 0.25) (layer B.Cu) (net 9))
 (segment (start 140.7 75.35) (end 138.9 75.35) (width 0.25) (layer B.Cu) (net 9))
 (segment (start 141.9 76.55) (end 140.7 75.35) (width 0.25) (layer B.Cu) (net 9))
 (segment (start 138.5 76.05) (end 138.5 75.4) (width 0.25) (layer B.Cu) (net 9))
 (segment (start 139 75.45) (end 139 76.05) (width 0.25) (layer B.Cu) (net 9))
 (segment (start 138.9 75.35) (end 139 75.45) (width 0.25) (layer B.Cu) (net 9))
 (segment (start 138.55 75.35) (end 138.9 75.35) (width 0.25) (layer B.Cu) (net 9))
 (segment (start 138.5 75.4) (end 138.55 75.35) (width 0.25) (layer B.Cu) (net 9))
 (segment (start 130.9 78.8) (end 132.95 78.8) (width 0.4) (layer B.Cu) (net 19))
 (segment (start 132.95 78.8) (end 133.5 78.25) (width 0.4) (layer B.Cu) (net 19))
 (segment (start 133.5 78.25) (end 133.85 78.25) (width 0.4) (layer B.Cu) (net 19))
 (segment (start 133.85 75.25) (end 134.7 75.25) (width 0.25) (layer B.Cu) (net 21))
 (segment (start 134.7 75.25) (end 135.7 74.25) (width 0.25) (layer B.Cu) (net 21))
 (segment (start 140.750002 74.35) (end 142.4 74.35) (width 0.25) (layer B.Cu) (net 21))
 (segment (start 140.650002 74.25) (end 140.750002 74.35) (width 0.25) (layer B.Cu) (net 21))
 (segment (start 135.7 74.25) (end 140.650002 74.25) (width 0.25) (layer B.Cu) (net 21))
 (segment (start 142.4 74.35) (end 142.6 74.55) (width 0.25) (layer B.Cu) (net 21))
 (segment (start 142.4 74.35) (end 142.6 74.55) (width 0.25) (layer B.Cu) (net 21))
 (segment (start 128.9 76.95) (end 127.08 76.95) (width 0.4) (layer B.Cu) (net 18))
 (segment (start 127.08 76.95) (end 126.44 77.59) (width 0.4) (layer B.Cu) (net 18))
 (segment (start 128.9 78.8) (end 127.77 78.8) (width 0.4) (layer B.Cu) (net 20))
 (segment (start 127.77 78.8) (end 126.44 80.13) (width 0.4) (layer B.Cu) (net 20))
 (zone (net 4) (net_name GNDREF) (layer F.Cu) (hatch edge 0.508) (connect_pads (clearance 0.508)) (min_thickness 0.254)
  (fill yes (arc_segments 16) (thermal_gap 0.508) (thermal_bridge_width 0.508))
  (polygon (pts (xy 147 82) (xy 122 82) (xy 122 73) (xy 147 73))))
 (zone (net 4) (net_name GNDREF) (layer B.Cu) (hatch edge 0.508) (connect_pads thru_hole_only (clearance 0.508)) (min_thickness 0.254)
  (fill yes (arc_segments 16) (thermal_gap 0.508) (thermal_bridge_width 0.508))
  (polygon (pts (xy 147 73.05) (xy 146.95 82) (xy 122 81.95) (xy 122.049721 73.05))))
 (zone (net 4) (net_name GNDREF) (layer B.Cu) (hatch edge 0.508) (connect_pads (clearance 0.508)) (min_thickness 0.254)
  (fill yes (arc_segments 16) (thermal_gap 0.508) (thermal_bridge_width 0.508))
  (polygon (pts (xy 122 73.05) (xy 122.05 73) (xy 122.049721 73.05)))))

